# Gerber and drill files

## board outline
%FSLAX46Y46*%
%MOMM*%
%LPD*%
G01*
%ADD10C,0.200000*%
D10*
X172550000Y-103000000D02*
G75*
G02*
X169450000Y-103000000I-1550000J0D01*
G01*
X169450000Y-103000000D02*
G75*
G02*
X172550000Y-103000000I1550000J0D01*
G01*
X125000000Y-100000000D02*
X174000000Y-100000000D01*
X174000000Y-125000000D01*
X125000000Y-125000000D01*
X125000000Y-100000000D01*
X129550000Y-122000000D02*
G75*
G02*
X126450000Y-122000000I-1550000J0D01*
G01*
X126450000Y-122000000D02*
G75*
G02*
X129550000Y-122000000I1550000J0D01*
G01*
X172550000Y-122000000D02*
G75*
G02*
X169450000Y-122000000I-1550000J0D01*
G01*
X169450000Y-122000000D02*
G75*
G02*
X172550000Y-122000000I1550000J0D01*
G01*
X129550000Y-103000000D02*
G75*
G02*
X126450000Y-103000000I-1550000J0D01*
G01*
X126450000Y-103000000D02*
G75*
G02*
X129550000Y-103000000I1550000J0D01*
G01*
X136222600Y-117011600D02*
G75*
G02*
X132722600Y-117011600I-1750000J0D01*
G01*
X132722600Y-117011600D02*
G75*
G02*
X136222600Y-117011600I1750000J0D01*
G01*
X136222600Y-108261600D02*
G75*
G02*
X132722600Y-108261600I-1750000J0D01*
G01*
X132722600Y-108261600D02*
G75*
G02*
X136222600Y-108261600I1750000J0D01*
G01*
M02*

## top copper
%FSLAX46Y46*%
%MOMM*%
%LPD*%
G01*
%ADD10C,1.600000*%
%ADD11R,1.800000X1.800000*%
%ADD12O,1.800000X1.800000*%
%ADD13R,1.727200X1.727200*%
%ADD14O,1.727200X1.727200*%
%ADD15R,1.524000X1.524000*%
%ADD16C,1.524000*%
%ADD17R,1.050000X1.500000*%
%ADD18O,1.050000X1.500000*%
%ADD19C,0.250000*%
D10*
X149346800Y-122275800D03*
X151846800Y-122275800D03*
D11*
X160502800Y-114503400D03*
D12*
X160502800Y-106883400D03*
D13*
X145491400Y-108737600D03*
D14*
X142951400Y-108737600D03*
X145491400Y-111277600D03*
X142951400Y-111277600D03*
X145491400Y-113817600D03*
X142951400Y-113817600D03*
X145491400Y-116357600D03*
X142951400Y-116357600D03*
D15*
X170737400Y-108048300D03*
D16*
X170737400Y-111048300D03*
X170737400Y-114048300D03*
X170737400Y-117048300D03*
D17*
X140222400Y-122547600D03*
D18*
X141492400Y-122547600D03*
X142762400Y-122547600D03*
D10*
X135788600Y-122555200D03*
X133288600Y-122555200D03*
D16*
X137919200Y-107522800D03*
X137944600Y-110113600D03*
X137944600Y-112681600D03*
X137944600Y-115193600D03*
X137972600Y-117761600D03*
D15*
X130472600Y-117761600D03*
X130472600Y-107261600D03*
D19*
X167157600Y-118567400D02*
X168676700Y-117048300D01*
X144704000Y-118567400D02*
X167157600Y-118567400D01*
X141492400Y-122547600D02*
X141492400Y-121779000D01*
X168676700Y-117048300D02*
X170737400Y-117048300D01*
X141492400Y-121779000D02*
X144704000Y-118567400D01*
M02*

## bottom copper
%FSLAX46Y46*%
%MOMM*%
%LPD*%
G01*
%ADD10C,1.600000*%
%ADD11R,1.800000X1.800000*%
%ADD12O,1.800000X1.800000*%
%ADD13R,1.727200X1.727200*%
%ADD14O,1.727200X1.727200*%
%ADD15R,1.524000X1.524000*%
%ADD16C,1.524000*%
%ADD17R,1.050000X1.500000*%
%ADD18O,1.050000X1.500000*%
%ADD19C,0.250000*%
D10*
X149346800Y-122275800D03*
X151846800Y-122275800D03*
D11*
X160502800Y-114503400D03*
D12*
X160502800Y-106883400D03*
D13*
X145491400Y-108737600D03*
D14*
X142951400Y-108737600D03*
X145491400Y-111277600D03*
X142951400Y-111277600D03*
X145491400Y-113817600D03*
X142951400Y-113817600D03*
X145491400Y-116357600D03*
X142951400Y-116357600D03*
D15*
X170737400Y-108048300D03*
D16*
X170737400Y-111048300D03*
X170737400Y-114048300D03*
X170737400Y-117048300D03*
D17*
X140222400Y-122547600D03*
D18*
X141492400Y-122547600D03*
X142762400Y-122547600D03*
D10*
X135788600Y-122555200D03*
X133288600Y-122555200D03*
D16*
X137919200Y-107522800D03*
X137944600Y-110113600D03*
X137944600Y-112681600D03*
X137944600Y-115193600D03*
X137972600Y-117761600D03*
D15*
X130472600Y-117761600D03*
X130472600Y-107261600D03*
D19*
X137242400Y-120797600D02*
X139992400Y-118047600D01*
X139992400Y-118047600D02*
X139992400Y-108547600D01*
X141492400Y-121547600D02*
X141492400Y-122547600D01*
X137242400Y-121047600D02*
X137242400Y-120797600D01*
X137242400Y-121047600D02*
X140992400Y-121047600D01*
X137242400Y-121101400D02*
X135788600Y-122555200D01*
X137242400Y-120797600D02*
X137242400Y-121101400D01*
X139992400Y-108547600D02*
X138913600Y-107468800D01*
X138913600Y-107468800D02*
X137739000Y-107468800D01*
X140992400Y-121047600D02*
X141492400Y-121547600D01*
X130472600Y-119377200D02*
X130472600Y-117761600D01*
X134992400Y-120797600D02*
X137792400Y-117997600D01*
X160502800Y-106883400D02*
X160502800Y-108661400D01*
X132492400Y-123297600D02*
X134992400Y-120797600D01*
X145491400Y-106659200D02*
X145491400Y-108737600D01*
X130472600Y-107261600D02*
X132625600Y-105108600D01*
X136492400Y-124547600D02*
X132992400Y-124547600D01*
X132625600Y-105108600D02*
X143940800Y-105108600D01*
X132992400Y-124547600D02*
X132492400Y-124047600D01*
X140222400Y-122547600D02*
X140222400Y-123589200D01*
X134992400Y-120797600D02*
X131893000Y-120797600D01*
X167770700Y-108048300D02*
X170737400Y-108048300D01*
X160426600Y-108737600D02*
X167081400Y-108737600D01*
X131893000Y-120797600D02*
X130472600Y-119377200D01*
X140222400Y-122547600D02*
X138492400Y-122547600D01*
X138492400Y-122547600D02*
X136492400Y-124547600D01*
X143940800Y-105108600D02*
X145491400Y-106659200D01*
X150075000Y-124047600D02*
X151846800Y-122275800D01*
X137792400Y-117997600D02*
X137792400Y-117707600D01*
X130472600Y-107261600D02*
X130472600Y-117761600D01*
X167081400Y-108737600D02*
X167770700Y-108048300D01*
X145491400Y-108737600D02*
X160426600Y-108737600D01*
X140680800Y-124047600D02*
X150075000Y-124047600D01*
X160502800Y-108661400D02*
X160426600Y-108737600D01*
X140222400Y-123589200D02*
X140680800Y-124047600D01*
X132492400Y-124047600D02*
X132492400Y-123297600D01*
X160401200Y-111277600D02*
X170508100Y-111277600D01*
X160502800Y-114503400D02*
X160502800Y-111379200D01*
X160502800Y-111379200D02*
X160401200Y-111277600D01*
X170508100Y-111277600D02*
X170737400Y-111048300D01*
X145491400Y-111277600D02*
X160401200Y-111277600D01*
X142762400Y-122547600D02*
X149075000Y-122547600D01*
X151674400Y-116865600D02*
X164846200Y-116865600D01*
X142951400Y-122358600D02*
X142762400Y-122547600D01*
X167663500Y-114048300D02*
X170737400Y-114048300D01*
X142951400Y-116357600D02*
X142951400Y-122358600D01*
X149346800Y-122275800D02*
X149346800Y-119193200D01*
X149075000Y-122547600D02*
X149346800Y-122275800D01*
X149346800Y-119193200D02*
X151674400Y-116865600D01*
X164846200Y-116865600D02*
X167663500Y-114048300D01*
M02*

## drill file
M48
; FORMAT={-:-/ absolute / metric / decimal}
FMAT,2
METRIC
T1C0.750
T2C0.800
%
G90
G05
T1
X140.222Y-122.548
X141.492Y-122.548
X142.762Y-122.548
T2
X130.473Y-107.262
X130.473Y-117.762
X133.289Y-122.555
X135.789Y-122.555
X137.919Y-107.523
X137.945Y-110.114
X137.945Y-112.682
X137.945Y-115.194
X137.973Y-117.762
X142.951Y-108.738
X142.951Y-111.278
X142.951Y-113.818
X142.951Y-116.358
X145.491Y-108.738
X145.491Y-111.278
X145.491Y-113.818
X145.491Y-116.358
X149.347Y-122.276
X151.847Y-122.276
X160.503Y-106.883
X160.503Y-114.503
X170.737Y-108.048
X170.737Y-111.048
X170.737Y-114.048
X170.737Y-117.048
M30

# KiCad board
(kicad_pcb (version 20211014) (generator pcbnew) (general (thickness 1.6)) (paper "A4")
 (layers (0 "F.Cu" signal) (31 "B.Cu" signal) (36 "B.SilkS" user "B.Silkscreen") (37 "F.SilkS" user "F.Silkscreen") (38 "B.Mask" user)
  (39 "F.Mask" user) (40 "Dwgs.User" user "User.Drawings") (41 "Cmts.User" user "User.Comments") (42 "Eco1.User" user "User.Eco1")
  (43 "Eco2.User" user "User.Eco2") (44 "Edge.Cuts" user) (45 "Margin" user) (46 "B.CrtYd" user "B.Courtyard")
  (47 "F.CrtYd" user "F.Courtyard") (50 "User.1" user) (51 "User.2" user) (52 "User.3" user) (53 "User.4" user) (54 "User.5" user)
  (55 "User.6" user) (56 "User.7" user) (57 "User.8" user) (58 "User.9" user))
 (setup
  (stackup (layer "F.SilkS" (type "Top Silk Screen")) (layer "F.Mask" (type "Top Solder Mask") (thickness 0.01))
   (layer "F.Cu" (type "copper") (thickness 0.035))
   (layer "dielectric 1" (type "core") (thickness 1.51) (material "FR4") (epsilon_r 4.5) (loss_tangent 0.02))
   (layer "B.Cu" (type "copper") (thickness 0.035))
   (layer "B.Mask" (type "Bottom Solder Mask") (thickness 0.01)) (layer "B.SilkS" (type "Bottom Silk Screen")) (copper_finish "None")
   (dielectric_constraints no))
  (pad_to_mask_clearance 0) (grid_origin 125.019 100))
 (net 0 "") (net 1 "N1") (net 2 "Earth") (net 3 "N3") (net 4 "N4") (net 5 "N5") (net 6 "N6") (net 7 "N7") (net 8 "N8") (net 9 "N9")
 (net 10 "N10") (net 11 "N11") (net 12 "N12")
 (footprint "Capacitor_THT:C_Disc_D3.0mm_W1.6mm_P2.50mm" (layer "F.Cu") (at 149.3468 122.2758)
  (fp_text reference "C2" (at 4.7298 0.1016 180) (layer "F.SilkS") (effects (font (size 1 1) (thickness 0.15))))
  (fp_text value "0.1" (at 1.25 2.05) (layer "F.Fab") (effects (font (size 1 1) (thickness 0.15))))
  (pad "1" thru_hole circle (at 0 0) (size 1.6 1.6) (drill 0.8) (layers *.Cu *.Mask) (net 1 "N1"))
  (pad "2" thru_hole circle (at 2.5 0) (size 1.6 1.6) (drill 0.8) (layers *.Cu *.Mask) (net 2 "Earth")))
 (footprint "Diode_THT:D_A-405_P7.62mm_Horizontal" (layer "F.Cu") (at 160.5028 114.5034 90)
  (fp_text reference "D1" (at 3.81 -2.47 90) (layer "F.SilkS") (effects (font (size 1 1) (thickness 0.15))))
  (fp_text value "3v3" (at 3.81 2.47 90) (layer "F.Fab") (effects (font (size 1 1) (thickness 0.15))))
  (pad "1" thru_hole rect (at 0 0 90) (size 1.8 1.8) (drill 0.8) (layers *.Cu *.Mask) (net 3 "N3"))
  (pad "2" thru_hole oval (at 7.62 0 90) (size 1.8 1.8) (drill 0.8) (layers *.Cu *.Mask) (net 2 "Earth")))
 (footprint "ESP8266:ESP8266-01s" (layer "F.Cu") (at 142.9514 108.7376)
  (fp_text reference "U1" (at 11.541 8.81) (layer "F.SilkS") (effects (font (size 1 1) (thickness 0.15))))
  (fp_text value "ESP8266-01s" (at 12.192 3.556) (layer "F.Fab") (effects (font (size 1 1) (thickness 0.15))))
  (pad "1" thru_hole rect (at 2.54 0) (size 1.7272 1.7272) (drill 0.8) (layers *.Cu *.Mask) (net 2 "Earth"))
  (pad "2" thru_hole oval (at 0 0) (size 1.7272 1.7272) (drill 0.8) (layers *.Cu *.Mask) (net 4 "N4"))
  (pad "3" thru_hole oval (at 2.54 2.54) (size 1.7272 1.7272) (drill 0.8) (layers *.Cu *.Mask) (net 3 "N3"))
  (pad "4" thru_hole oval (at 0 2.54) (size 1.7272 1.7272) (drill 0.8) (layers *.Cu *.Mask) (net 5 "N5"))
  (pad "5" thru_hole oval (at 2.54 5.08) (size 1.7272 1.7272) (drill 0.8) (layers *.Cu *.Mask) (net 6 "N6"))
  (pad "6" thru_hole oval (at 0 5.08) (size 1.7272 1.7272) (drill 0.8) (layers *.Cu *.Mask) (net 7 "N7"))
  (pad "7" thru_hole oval (at 2.54 7.62) (size 1.7272 1.7272) (drill 0.8) (layers *.Cu *.Mask) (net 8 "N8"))
  (pad "8" thru_hole oval (at 0 7.62) (size 1.7272 1.7272) (drill 0.8) (layers *.Cu *.Mask) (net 1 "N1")))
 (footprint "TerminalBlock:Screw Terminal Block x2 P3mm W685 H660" (layer "F.Cu") (at 170.7374 108.0483 -90)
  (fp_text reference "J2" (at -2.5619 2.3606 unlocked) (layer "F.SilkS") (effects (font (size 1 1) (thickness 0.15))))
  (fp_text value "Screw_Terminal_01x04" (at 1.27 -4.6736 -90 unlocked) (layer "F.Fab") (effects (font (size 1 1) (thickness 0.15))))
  (pad "1" thru_hole rect (at 0 0 270) (size 1.524 1.524) (drill 0.8) (layers *.Cu *.Mask) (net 2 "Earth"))
  (pad "2" thru_hole circle (at 3 0 270) (size 1.524 1.524) (drill 0.8) (layers *.Cu *.Mask) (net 3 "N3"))
  (pad "3" thru_hole circle (at 6 0 270) (size 1.524 1.524) (drill 0.8) (layers *.Cu *.Mask) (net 1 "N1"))
  (pad "4" thru_hole circle (at 9 0 270) (size 1.524 1.524) (drill 0.8) (layers *.Cu *.Mask) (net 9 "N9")))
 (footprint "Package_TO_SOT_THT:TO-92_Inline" (layer "F.Cu") (at 140.2224 122.5476)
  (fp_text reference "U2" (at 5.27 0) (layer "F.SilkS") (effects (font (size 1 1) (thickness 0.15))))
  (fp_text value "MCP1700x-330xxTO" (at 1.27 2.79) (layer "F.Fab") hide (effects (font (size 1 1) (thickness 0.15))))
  (pad "1" thru_hole rect (at 0 0) (size 1.05 1.5) (drill 0.75) (layers *.Cu *.Mask) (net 2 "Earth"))
  (pad "2" thru_hole oval (at 1.27 0) (size 1.05 1.5) (drill 0.75) (layers *.Cu *.Mask) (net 9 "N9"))
  (pad "3" thru_hole oval (at 2.54 0) (size 1.05 1.5) (drill 0.75) (layers *.Cu *.Mask) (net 1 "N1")))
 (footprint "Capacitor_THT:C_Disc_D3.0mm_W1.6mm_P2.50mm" (layer "F.Cu") (at 135.7886 122.5552 180)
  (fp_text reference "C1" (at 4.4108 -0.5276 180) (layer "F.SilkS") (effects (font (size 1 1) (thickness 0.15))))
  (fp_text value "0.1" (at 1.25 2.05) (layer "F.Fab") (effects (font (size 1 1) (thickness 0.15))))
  (pad "1" thru_hole circle (at 0 0 180) (size 1.6 1.6) (drill 0.8) (layers *.Cu *.Mask) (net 9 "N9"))
  (pad "2" thru_hole circle (at 2.5 0 180) (size 1.6 1.6) (drill 0.8) (layers *.Cu *.Mask) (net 2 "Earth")))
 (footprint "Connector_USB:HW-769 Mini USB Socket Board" (layer "F.Cu") (at 139.7226 119.5116)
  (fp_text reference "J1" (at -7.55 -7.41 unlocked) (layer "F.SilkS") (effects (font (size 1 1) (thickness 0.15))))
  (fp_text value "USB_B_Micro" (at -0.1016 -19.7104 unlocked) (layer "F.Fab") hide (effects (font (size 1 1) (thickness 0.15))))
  (fp_circle (center -5.25 -2.5) (end -3.5 -2.5) (layer "Edge.Cuts") (width 0.2) (fill none))
  (fp_circle (center -5.25 -11.25) (end -3.5 -11.25) (layer "Edge.Cuts") (width 0.2) (fill none))
  (pad "1" thru_hole circle (at -1.8034 -11.9888) (size 1.524 1.524) (drill 0.8) (layers *.Cu *.Mask) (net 9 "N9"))
  (pad "2" thru_hole circle (at -1.778 -9.398) (size 1.524 1.524) (drill 0.8) (layers *.Cu *.Mask) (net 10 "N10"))
  (pad "3" thru_hole circle (at -1.778 -6.83) (size 1.524 1.524) (drill 0.8) (layers *.Cu *.Mask) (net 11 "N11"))
  (pad "4" thru_hole circle (at -1.778 -4.318) (size 1.524 1.524) (drill 0.8) (layers *.Cu *.Mask) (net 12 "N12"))
  (pad "5" thru_hole circle (at -1.75 -1.75) (size 1.524 1.524) (drill 0.8) (layers *.Cu *.Mask) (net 2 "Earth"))
  (pad "6" thru_hole rect (at -9.25 -1.75) (size 1.524 1.524) (drill 0.8) (layers *.Cu *.Mask) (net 2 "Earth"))
  (pad "7" thru_hole rect (at -9.25 -12.25) (size 1.524 1.524) (drill 0.8) (layers *.Cu *.Mask) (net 2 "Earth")))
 (gr_circle (center 171 103) (end 172.55 103) (layer "Edge.Cuts") (width 0.2) (fill none))
 (gr_rect (start 125 100) (end 174 125) (layer "Edge.Cuts") (width 0.2) (fill none))
 (gr_circle (center 128 122) (end 129.55 122) (layer "Edge.Cuts") (width 0.2) (fill none))
 (gr_circle (center 171 122) (end 172.55 122) (layer "Edge.Cuts") (width 0.2) (fill none))
 (gr_circle (center 128 103) (end 129.55 103) (layer "Edge.Cuts") (width 0.2) (fill none))
 (segment (start 167.1576 118.5674) (end 168.6767 117.0483) (width 0.25) (layer "F.Cu") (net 9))
 (segment (start 144.704 118.5674) (end 167.1576 118.5674) (width 0.25) (layer "F.Cu") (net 9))
 (segment (start 141.4924 122.5476) (end 141.4924 121.779) (width 0.25) (layer "F.Cu") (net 9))
 (segment (start 168.6767 117.0483) (end 170.7374 117.0483) (width 0.25) (layer "F.Cu") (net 9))
 (segment (start 141.4924 121.779) (end 144.704 118.5674) (width 0.25) (layer "F.Cu") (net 9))
 (segment (start 137.2424 120.7976) (end 139.9924 118.0476) (width 0.25) (layer "B.Cu") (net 9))
 (segment (start 139.9924 118.0476) (end 139.9924 108.5476) (width 0.25) (layer "B.Cu") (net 9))
 (segment (start 141.4924 121.5476) (end 141.4924 122.5476) (width 0.25) (layer "B.Cu") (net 9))
 (segment (start 137.2424 121.0476) (end 137.2424 120.7976) (width 0.25) (layer "B.Cu") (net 9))
 (segment (start 137.2424 121.0476) (end 140.9924 121.0476) (width 0.25) (layer "B.Cu") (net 9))
 (segment (start 137.2424 121.1014) (end 135.7886 122.5552) (width 0.25) (layer "B.Cu") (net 9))
 (segment (start 137.2424 120.7976) (end 137.2424 121.1014) (width 0.25) (layer "B.Cu") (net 9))
 (segment (start 139.9924 108.5476) (end 138.9136 107.4688) (width 0.25) (layer "B.Cu") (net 9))
 (segment (start 138.9136 107.4688) (end 137.739 107.4688) (width 0.25) (layer "B.Cu") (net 9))
 (segment (start 140.9924 121.0476) (end 141.4924 121.5476) (width 0.25) (layer "B.Cu") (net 9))
 (segment (start 130.4726 119.3772) (end 130.4726 117.7616) (width 0.25) (layer "B.Cu") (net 2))
 (segment (start 134.9924 120.7976) (end 137.7924 117.9976) (width 0.25) (layer "B.Cu") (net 2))
 (segment (start 160.5028 106.8834) (end 160.5028 108.6614) (width 0.25) (layer "B.Cu") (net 2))
 (segment (start 132.4924 123.2976) (end 134.9924 120.7976) (width 0.25) (layer "B.Cu") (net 2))
 (segment (start 145.4914 106.6592) (end 145.4914 108.7376) (width 0.25) (layer "B.Cu") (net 2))
 (segment (start 130.4726 107.2616) (end 132.6256 105.1086) (width 0.25) (layer "B.Cu") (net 2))
 (segment (start 136.4924 124.5476) (end 132.9924 124.5476) (width 0.25) (layer "B.Cu") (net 2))
 (segment (start 132.6256 105.1086) (end 143.9408 105.1086) (width 0.25) (layer "B.Cu") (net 2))
 (segment (start 132.9924 124.5476) (end 132.4924 124.0476) (width 0.25) (layer "B.Cu") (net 2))
 (segment (start 140.2224 122.5476) (end 140.2224 123.5892) (width 0.25) (layer "B.Cu") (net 2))
 (segment (start 134.9924 120.7976) (end 131.893 120.7976) (width 0.25) (layer "B.Cu") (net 2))
 (segment (start 167.7707 108.0483) (end 170.7374 108.0483) (width 0.25) (layer "B.Cu") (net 2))
 (segment (start 160.4266 108.7376) (end 167.0814 108.7376) (width 0.25) (layer "B.Cu") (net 2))
 (segment (start 131.893 120.7976) (end 130.4726 119.3772) (width 0.25) (layer "B.Cu") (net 2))
 (segment (start 140.2224 122.5476) (end 138.4924 122.5476) (width 0.25) (layer "B.Cu") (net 2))
 (segment (start 138.4924 122.5476) (end 136.4924 124.5476) (width 0.25) (layer "B.Cu") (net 2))
 (segment (start 143.9408 105.1086) (end 145.4914 106.6592) (width 0.25) (layer "B.Cu") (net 2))
 (segment (start 150.075 124.0476) (end 151.8468 122.2758) (width 0.25) (layer "B.Cu") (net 2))
 (segment (start 137.7924 117.9976) (end 137.7924 117.7076) (width 0.25) (layer "B.Cu") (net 2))
 (segment (start 130.4726 107.2616) (end 130.4726 117.7616) (width 0.25) (layer "B.Cu") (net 2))
 (segment (start 167.0814 108.7376) (end 167.7707 108.0483) (width 0.25) (layer "B.Cu") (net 2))
 (segment (start 145.4914 108.7376) (end 160.4266 108.7376) (width 0.25) (layer "B.Cu") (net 2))
 (segment (start 140.6808 124.0476) (end 150.075 124.0476) (width 0.25) (layer "B.Cu") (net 2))
 (segment (start 160.5028 108.6614) (end 160.4266 108.7376) (width 0.25) (layer "B.Cu") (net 2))
 (segment (start 140.2224 123.5892) (end 140.6808 124.0476) (width 0.25) (layer "B.Cu") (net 2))
 (segment (start 132.4924 124.0476) (end 132.4924 123.2976) (width 0.25) (layer "B.Cu") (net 2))
 (segment (start 160.4012 111.2776) (end 170.5081 111.2776) (width 0.25) (layer "B.Cu") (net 3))
 (segment (start 160.5028 114.5034) (end 160.5028 111.3792) (width 0.25) (layer "B.Cu") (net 3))
 (segment (start 160.5028 111.3792) (end 160.4012 111.2776) (width 0.25) (layer "B.Cu") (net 3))
 (segment (start 170.5081 111.2776) (end 170.7374 111.0483) (width 0.25) (layer "B.Cu") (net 3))
 (segment (start 145.4914 111.2776) (end 160.4012 111.2776) (width 0.25) (layer "B.Cu") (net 3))
 (segment (start 142.7624 122.5476) (end 149.075 122.5476) (width 0.25) (layer "B.Cu") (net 1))
 (segment (start 151.6744 116.8656) (end 164.8462 116.8656) (width 0.25) (layer "B.Cu") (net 1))
 (segment (start 142.9514 122.3586) (end 142.7624 122.5476) (width 0.25) (layer "B.Cu") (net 1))
 (segment (start 167.6635 114.0483) (end 170.7374 114.0483) (width 0.25) (layer "B.Cu") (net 1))
 (segment (start 142.9514 116.3576) (end 142.9514 122.3586) (width 0.25) (layer "B.Cu") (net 1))
 (segment (start 149.3468 122.2758) (end 149.3468 119.1932) (width 0.25) (layer "B.Cu") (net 1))
 (segment (start 149.075 122.5476) (end 149.3468 122.2758) (width 0.25) (layer "B.Cu") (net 1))
 (segment (start 149.3468 119.1932) (end 151.6744 116.8656) (width 0.25) (layer "B.Cu") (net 1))
 (segment (start 164.8462 116.8656) (end 167.6635 114.0483) (width 0.25) (layer "B.Cu") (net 1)))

